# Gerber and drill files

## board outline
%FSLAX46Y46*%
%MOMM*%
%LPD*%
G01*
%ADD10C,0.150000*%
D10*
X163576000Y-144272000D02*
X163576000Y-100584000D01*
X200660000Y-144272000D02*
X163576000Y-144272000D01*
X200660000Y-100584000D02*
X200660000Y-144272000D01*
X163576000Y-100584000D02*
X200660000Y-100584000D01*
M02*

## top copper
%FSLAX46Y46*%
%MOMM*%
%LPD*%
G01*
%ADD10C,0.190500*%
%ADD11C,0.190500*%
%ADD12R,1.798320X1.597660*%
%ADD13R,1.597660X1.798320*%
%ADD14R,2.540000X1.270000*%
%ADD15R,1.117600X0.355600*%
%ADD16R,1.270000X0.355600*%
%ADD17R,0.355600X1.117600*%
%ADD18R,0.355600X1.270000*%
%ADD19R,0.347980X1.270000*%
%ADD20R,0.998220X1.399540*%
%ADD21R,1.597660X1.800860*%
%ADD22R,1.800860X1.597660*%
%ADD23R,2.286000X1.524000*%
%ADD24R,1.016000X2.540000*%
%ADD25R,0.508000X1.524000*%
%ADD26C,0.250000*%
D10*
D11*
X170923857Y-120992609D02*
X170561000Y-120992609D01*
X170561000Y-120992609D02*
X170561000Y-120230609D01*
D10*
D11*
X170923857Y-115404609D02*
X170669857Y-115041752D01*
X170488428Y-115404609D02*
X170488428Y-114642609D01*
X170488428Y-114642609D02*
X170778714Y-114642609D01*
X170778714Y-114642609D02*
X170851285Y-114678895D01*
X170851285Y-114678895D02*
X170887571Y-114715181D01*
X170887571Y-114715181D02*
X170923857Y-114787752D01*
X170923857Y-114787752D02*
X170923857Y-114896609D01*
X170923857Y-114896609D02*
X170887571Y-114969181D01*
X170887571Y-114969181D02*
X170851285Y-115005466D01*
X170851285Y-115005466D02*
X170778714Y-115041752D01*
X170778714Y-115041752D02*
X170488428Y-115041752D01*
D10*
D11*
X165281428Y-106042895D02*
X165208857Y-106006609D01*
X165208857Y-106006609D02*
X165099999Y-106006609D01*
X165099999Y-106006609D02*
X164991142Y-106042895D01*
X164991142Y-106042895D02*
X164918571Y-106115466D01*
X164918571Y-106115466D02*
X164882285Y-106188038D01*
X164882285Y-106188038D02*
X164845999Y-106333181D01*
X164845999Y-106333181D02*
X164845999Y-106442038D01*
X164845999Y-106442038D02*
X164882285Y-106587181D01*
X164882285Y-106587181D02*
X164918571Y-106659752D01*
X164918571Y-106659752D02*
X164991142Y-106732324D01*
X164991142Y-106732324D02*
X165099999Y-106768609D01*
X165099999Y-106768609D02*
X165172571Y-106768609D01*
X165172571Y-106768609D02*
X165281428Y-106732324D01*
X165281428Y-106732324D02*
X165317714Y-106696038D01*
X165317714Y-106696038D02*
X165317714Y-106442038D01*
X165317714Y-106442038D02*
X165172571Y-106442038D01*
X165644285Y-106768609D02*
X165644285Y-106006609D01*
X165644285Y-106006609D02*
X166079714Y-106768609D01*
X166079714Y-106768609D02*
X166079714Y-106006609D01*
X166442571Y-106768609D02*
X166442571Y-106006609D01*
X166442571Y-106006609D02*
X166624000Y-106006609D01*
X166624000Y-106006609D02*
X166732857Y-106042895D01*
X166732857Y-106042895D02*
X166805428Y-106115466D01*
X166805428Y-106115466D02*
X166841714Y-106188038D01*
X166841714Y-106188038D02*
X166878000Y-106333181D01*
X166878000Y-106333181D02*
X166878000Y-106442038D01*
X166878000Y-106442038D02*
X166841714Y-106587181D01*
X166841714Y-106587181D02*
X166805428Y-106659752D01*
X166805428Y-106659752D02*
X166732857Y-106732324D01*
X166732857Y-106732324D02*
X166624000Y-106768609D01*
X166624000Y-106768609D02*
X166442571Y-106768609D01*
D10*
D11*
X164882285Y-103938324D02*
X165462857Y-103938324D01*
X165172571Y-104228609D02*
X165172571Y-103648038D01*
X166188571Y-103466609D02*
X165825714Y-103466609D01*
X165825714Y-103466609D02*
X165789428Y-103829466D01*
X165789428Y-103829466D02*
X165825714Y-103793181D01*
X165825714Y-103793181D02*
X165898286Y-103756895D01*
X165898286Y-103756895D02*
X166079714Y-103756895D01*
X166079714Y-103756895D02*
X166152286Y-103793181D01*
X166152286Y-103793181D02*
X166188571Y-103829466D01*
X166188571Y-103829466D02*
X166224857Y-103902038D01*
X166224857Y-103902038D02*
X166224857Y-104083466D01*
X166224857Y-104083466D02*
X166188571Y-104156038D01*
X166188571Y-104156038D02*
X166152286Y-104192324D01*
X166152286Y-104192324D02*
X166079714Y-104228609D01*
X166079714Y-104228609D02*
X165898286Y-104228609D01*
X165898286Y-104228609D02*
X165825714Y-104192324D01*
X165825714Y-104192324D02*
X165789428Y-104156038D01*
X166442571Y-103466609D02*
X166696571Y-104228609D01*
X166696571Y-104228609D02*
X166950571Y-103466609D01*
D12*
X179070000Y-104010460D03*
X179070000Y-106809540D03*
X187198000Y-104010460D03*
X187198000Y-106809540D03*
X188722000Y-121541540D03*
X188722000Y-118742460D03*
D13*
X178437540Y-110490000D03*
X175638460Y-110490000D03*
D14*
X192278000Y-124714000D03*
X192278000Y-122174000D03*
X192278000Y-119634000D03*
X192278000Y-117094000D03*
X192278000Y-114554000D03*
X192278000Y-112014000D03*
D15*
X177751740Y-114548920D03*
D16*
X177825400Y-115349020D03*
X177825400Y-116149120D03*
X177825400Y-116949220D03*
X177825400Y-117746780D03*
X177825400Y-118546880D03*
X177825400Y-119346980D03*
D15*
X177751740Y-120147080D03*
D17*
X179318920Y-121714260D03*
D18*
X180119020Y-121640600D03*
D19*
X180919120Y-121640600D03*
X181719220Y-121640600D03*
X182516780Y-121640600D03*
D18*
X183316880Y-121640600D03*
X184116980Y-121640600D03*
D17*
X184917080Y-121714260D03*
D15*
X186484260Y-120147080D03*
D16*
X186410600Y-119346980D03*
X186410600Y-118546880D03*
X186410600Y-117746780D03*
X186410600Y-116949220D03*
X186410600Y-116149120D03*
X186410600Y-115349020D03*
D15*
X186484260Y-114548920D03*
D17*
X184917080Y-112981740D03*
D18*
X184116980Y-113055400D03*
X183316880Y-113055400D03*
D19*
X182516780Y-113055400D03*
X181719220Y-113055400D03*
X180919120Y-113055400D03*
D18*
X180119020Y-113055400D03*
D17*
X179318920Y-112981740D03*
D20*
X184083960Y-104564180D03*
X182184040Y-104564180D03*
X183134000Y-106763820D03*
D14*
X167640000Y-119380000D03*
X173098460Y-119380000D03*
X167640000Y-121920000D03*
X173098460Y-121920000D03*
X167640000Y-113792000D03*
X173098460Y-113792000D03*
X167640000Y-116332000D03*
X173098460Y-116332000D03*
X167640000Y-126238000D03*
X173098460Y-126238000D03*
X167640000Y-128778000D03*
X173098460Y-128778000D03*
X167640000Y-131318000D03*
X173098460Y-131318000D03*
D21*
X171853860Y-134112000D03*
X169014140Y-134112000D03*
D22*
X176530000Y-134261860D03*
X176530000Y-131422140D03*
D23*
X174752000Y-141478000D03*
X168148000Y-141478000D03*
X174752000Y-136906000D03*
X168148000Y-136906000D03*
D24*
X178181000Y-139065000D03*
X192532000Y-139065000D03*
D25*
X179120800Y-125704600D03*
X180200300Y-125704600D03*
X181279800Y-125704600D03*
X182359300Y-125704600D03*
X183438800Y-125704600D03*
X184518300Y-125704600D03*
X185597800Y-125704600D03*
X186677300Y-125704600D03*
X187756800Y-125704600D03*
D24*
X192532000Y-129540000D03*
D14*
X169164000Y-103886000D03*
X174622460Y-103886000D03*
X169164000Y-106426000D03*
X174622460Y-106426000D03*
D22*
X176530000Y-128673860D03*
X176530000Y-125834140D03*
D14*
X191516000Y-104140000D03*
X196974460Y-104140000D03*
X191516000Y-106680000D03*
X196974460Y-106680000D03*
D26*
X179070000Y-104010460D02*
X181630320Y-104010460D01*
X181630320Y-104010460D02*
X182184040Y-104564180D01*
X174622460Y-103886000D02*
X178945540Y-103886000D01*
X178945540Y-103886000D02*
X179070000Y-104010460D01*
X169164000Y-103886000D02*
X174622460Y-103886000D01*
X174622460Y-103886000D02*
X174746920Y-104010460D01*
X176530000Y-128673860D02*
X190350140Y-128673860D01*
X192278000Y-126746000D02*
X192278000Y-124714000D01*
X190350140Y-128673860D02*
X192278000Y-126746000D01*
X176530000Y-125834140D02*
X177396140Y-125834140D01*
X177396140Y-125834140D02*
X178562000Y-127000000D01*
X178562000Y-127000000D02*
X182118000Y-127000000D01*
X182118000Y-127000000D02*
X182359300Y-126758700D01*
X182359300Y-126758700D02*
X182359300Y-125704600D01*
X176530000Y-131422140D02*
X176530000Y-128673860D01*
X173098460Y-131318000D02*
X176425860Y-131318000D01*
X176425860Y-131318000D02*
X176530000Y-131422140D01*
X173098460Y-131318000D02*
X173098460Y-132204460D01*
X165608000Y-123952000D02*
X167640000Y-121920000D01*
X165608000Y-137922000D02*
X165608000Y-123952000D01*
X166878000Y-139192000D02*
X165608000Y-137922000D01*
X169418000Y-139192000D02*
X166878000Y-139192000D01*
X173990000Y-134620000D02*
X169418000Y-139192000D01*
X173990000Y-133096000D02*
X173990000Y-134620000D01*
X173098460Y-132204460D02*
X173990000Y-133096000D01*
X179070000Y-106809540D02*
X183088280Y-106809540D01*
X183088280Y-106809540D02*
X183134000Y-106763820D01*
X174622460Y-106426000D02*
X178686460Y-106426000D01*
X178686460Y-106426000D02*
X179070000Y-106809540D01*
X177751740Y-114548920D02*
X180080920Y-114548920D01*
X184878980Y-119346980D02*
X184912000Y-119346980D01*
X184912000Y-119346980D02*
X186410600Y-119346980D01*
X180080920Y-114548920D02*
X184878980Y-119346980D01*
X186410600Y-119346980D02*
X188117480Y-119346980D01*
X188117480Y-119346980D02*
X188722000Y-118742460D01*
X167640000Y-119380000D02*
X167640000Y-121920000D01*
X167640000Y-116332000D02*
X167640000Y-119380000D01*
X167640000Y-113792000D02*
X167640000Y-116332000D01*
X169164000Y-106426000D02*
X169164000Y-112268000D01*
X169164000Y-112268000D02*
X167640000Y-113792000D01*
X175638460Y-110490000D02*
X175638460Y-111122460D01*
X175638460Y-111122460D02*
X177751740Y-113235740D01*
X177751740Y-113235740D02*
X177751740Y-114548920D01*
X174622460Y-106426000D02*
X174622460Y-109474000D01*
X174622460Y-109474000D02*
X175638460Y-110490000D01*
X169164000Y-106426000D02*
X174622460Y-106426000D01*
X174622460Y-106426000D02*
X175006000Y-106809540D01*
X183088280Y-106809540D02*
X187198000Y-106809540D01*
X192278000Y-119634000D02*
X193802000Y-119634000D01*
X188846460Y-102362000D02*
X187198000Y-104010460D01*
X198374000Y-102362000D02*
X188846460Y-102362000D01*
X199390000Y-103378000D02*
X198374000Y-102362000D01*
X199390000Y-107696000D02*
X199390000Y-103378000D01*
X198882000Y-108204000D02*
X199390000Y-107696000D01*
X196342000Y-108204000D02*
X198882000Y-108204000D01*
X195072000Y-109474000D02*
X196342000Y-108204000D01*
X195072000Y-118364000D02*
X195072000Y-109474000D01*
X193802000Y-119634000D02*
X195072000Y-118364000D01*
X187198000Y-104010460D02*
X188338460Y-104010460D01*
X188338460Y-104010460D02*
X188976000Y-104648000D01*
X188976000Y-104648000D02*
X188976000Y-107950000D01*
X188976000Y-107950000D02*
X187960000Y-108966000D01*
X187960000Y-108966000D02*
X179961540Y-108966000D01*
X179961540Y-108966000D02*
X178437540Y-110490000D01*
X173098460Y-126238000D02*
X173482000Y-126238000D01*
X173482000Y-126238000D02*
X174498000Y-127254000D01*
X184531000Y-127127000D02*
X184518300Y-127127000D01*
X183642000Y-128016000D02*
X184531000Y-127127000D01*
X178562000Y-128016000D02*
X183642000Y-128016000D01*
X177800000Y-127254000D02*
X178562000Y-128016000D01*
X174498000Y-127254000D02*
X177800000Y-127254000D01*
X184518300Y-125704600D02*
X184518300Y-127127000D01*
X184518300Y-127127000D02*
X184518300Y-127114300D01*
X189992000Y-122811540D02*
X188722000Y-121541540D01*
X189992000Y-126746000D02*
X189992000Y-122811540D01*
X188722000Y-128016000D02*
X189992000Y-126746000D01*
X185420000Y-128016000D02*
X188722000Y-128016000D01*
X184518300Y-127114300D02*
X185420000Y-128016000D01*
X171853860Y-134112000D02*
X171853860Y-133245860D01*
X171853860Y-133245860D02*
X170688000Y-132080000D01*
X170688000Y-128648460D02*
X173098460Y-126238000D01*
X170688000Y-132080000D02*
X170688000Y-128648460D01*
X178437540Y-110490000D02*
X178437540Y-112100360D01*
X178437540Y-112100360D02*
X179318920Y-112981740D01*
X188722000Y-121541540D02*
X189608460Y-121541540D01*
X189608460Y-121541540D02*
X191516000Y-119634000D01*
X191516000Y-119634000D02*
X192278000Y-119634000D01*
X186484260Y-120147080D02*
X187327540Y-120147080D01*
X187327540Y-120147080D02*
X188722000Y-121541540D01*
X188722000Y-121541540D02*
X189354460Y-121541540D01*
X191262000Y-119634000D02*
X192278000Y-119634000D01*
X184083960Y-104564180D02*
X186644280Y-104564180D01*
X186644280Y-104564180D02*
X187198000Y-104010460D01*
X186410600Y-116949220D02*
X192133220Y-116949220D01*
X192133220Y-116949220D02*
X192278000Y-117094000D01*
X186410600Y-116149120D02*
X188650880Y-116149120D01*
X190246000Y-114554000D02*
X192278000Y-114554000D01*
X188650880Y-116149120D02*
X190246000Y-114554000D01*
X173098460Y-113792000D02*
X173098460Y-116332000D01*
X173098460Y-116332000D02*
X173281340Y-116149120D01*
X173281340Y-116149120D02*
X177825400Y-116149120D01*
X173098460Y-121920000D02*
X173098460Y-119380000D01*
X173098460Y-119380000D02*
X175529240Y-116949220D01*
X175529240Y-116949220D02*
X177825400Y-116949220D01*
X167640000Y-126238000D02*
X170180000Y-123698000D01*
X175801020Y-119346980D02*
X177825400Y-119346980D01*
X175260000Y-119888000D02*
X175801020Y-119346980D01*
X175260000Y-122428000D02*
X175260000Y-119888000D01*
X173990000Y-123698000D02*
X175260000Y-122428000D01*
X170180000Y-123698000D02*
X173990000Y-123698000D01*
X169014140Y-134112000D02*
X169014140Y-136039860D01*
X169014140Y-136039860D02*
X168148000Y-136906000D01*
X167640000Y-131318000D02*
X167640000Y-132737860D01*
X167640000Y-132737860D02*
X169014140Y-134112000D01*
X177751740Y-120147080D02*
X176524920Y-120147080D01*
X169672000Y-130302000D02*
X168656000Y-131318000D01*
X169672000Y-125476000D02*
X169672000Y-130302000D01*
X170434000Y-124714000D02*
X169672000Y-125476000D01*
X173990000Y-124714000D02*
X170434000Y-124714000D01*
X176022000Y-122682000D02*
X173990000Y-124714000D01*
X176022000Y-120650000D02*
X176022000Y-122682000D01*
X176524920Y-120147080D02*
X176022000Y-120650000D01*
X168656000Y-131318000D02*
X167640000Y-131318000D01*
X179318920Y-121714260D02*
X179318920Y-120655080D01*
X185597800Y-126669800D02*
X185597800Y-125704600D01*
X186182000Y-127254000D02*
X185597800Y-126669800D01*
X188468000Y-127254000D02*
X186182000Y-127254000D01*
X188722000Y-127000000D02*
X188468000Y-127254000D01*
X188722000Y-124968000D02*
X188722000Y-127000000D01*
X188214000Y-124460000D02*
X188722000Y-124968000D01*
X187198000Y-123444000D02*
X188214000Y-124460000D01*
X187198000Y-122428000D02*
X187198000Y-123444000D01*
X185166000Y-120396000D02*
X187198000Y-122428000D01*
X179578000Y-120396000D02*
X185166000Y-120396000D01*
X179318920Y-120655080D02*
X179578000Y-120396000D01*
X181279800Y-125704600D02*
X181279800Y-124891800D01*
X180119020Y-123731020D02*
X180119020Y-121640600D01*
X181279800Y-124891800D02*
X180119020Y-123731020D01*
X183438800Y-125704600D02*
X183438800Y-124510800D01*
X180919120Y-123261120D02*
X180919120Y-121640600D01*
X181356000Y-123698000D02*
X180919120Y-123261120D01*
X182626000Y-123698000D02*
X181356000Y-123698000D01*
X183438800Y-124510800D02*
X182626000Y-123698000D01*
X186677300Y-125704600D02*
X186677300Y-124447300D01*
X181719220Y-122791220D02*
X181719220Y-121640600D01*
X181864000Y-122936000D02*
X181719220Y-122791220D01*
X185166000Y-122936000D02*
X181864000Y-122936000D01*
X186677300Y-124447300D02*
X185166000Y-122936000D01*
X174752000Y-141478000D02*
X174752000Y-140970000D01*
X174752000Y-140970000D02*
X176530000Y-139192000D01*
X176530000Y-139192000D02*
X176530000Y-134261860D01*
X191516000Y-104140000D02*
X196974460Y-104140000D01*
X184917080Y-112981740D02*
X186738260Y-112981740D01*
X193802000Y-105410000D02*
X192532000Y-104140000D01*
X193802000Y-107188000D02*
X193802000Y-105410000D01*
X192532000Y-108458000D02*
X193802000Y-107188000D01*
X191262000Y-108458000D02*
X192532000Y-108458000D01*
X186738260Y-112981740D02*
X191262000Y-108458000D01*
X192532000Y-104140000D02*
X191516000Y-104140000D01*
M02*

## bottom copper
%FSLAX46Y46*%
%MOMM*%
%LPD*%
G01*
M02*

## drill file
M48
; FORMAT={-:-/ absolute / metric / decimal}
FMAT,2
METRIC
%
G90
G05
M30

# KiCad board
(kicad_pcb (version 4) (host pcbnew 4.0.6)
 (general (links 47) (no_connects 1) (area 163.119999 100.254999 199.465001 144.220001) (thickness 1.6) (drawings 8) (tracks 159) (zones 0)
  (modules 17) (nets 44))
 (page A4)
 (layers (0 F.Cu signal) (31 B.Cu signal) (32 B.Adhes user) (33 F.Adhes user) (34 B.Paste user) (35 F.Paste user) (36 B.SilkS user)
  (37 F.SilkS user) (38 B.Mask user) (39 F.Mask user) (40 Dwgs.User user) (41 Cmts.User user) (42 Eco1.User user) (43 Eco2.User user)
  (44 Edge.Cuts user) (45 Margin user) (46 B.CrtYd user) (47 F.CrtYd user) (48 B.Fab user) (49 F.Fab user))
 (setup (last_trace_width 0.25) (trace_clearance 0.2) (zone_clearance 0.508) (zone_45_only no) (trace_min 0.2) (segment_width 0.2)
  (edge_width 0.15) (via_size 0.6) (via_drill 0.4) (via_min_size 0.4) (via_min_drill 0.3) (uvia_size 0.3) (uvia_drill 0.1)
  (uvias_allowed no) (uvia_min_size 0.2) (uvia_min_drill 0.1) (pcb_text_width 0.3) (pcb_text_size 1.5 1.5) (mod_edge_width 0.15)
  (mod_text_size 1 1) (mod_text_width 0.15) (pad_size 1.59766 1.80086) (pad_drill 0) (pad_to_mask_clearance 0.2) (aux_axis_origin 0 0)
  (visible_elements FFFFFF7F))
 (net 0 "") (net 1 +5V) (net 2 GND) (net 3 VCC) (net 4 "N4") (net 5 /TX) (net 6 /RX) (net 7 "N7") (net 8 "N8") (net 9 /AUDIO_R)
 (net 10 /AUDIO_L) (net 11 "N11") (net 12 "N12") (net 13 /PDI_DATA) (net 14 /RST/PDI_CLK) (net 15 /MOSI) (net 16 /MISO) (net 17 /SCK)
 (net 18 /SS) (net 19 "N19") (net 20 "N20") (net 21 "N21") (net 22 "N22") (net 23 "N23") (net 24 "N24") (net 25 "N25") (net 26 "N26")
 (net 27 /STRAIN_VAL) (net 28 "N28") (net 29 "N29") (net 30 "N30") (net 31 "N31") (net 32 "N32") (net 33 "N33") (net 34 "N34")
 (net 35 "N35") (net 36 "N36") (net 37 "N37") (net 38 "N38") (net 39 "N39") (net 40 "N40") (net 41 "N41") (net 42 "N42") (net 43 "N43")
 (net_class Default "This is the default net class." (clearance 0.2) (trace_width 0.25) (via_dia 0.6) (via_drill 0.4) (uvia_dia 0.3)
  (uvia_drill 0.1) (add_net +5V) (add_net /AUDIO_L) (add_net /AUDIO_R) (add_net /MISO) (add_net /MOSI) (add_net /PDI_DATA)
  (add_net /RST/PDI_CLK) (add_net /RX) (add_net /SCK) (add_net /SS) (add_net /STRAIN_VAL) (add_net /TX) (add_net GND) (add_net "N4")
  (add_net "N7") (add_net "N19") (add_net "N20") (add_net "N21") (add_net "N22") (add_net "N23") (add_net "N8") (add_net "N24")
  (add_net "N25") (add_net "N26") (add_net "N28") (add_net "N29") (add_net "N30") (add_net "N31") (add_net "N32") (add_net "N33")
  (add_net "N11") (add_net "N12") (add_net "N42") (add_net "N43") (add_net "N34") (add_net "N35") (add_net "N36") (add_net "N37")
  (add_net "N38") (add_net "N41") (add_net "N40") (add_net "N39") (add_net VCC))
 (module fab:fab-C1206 (layer F.Cu) (at 179.07 105.41 270)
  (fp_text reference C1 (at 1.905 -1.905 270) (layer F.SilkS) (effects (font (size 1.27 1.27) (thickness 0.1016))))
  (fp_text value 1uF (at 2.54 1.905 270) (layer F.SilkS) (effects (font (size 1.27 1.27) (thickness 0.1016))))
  (pad 1 smd rect (at -1.39954 0 270) (size 1.59766 1.79832) (layers F.Cu F.Paste F.Mask) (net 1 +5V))
  (pad 2 smd rect (at 1.39954 0 270) (size 1.59766 1.79832) (layers F.Cu F.Paste F.Mask) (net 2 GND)))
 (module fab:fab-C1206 (layer F.Cu) (at 187.198 105.41 270)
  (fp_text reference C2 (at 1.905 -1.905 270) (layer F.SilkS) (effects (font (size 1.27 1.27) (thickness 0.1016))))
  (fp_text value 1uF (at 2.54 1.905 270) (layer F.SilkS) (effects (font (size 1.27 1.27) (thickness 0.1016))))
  (pad 1 smd rect (at -1.39954 0 270) (size 1.59766 1.79832) (layers F.Cu F.Paste F.Mask) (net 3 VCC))
  (pad 2 smd rect (at 1.39954 0 270) (size 1.59766 1.79832) (layers F.Cu F.Paste F.Mask) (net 2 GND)))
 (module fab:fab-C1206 (layer F.Cu) (at 188.722 120.142 90)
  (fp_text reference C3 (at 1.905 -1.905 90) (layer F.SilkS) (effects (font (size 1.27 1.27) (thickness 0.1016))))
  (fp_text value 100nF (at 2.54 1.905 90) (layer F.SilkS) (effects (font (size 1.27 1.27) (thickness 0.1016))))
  (pad 1 smd rect (at -1.39954 0 90) (size 1.59766 1.79832) (layers F.Cu F.Paste F.Mask) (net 3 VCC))
  (pad 2 smd rect (at 1.39954 0 90) (size 1.59766 1.79832) (layers F.Cu F.Paste F.Mask) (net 2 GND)))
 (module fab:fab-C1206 (layer F.Cu) (at 177.038 110.49 180)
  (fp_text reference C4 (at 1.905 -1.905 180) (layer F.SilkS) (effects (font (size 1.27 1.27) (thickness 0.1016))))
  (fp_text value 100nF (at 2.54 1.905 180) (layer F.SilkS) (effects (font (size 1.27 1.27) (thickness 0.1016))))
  (pad 1 smd rect (at -1.39954 0 180) (size 1.59766 1.79832) (layers F.Cu F.Paste F.Mask) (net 3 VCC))
  (pad 2 smd rect (at 1.39954 0 180) (size 1.59766 1.79832) (layers F.Cu F.Paste F.Mask) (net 2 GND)))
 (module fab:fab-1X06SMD (layer F.Cu) (at 192.278 118.364 180)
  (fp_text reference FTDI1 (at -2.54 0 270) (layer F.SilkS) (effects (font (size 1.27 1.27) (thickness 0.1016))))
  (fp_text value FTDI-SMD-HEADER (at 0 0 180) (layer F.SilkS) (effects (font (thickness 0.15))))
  (pad 1 smd rect (at 0 -6.35 180) (size 2.54 1.27) (layers F.Cu F.Paste F.Mask) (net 2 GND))
  (pad 2 smd rect (at 0 -3.81 180) (size 2.54 1.27) (layers F.Cu F.Paste F.Mask) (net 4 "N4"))
  (pad 3 smd rect (at 0 -1.27 180) (size 2.54 1.27) (layers F.Cu F.Paste F.Mask) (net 3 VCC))
  (pad 4 smd rect (at 0 1.27 180) (size 2.54 1.27) (layers F.Cu F.Paste F.Mask) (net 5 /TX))
  (pad 5 smd rect (at 0 3.81 180) (size 2.54 1.27) (layers F.Cu F.Paste F.Mask) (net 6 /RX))
  (pad 6 smd rect (at 0 6.35 180) (size 2.54 1.27) (layers F.Cu F.Paste F.Mask) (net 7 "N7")))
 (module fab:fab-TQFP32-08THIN (layer F.Cu) (at 182.118 117.348)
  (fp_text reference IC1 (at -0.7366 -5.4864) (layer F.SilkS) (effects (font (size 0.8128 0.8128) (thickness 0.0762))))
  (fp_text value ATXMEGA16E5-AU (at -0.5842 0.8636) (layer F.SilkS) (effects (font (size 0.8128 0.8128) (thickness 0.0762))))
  (pad 1 smd rect (at -4.36626 -2.79908) (size 1.1176 0.3556) (layers F.Cu F.Paste F.Mask) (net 2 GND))
  (pad 2 smd rect (at -4.2926 -1.99898) (size 1.27 0.3556) (layers F.Cu F.Paste F.Mask) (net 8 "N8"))
  (pad 3 smd rect (at -4.2926 -1.19888) (size 1.27 0.3556) (layers F.Cu F.Paste F.Mask) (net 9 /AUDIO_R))
  (pad 4 smd rect (at -4.2926 -0.39878) (size 1.27 0.3556) (layers F.Cu F.Paste F.Mask) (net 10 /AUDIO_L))
  (pad 5 smd rect (at -4.2926 0.39878) (size 1.27 0.3556) (layers F.Cu F.Paste F.Mask) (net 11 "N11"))
  (pad 6 smd rect (at -4.2926 1.19888) (size 1.27 0.3556) (layers F.Cu F.Paste F.Mask) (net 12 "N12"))
  (pad 7 smd rect (at -4.2926 1.99898) (size 1.27 0.3556) (layers F.Cu F.Paste F.Mask) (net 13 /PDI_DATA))
  (pad 8 smd rect (at -4.36626 2.79908) (size 1.1176 0.3556) (layers F.Cu F.Paste F.Mask) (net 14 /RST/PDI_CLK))
  (pad 9 smd rect (at -2.79908 4.36626) (size 0.3556 1.1176) (layers F.Cu F.Paste F.Mask) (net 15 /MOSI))
  (pad 10 smd rect (at -1.99898 4.2926) (size 0.3556 1.27) (layers F.Cu F.Paste F.Mask) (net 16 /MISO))
  (pad 11 smd rect (at -1.19888 4.2926) (size 0.34798 1.27) (layers F.Cu F.Paste F.Mask) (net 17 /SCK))
  (pad 12 smd rect (at -0.39878 4.2926) (size 0.34798 1.27) (layers F.Cu F.Paste F.Mask) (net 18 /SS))
  (pad 13 smd rect (at 0.39878 4.2926) (size 0.34798 1.27) (layers F.Cu F.Paste F.Mask) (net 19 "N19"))
  (pad 14 smd rect (at 1.19888 4.2926) (size 0.3556 1.27) (layers F.Cu F.Paste F.Mask) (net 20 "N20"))
  (pad 15 smd rect (at 1.99898 4.2926) (size 0.3556 1.27) (layers F.Cu F.Paste F.Mask) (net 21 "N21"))
  (pad 16 smd rect (at 2.79908 4.36626) (size 0.3556 1.1176) (layers F.Cu F.Paste F.Mask) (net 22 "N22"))
  (pad 17 smd rect (at 4.36626 2.79908) (size 1.1176 0.3556) (layers F.Cu F.Paste F.Mask) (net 3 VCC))
  (pad 18 smd rect (at 4.2926 1.99898) (size 1.27 0.3556) (layers F.Cu F.Paste F.Mask) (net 2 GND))
  (pad 19 smd rect (at 4.2926 1.19888) (size 1.27 0.3556) (layers F.Cu F.Paste F.Mask) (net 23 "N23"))
  (pad 20 smd rect (at 4.2926 0.39878) (size 1.27 0.3556) (layers F.Cu F.Paste F.Mask) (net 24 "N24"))
  (pad 21 smd rect (at 4.2926 -0.39878) (size 1.27 0.3556) (layers F.Cu F.Paste F.Mask) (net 5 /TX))
  (pad 22 smd rect (at 4.2926 -1.19888) (size 1.27 0.3556) (layers F.Cu F.Paste F.Mask) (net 6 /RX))
  (pad 23 smd rect (at 4.2926 -1.99898) (size 1.27 0.3556) (layers F.Cu F.Paste F.Mask) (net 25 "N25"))
  (pad 24 smd rect (at 4.36626 -2.79908) (size 1.1176 0.3556) (layers F.Cu F.Paste F.Mask) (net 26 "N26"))
  (pad 25 smd rect (at 2.79908 -4.36626) (size 0.3556 1.1176) (layers F.Cu F.Paste F.Mask) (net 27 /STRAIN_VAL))
  (pad 26 smd rect (at 1.99898 -4.2926) (size 0.3556 1.27) (layers F.Cu F.Paste F.Mask) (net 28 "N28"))
  (pad 27 smd rect (at 1.19888 -4.2926) (size 0.3556 1.27) (layers F.Cu F.Paste F.Mask) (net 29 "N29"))
  (pad 28 smd rect (at 0.39878 -4.2926) (size 0.34798 1.27) (layers F.Cu F.Paste F.Mask) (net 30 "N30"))
  (pad 29 smd rect (at -0.39878 -4.2926) (size 0.34798 1.27) (layers F.Cu F.Paste F.Mask) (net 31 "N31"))
  (pad 30 smd rect (at -1.19888 -4.2926) (size 0.34798 1.27) (layers F.Cu F.Paste F.Mask) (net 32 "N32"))
  (pad 31 smd rect (at -1.99898 -4.2926) (size 0.3556 1.27) (layers F.Cu F.Paste F.Mask) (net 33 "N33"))
  (pad 32 smd rect (at -2.79908 -4.36626) (size 0.3556 1.1176) (layers F.Cu F.Paste F.Mask) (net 3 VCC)))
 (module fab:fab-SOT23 (layer F.Cu) (at 183.134 105.664 180)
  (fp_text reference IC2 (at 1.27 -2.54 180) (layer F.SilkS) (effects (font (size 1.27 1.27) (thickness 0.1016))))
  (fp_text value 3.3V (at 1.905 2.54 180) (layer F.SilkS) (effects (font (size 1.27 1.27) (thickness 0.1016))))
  (pad 1 smd rect (at -0.94996 1.09982 180) (size 0.99822 1.39954) (layers F.Cu F.Paste F.Mask) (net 3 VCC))
  (pad 2 smd rect (at 0.94996 1.09982 180) (size 0.99822 1.39954) (layers F.Cu F.Paste F.Mask) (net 1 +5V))
  (pad 3 smd rect (at 0 -1.09982 180) (size 0.99822 1.39954) (layers F.Cu F.Paste F.Mask) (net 2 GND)))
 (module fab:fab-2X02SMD (layer F.Cu) (at 170.18 120.65)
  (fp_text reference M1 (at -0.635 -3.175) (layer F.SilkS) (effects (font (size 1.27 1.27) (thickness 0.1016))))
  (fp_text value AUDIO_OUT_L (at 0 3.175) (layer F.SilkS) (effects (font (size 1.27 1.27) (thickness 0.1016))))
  (pad 1 smd rect (at -2.54 -1.27) (size 2.54 1.27) (layers F.Cu F.Paste F.Mask) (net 2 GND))
  (pad 2 smd rect (at 2.91846 -1.27) (size 2.54 1.27) (layers F.Cu F.Paste F.Mask) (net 10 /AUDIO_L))
  (pad 3 smd rect (at -2.54 1.27) (size 2.54 1.27) (layers F.Cu F.Paste F.Mask) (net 2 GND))
  (pad 4 smd rect (at 2.91846 1.27) (size 2.54 1.27) (layers F.Cu F.Paste F.Mask) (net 10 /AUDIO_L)))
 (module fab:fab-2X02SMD (layer F.Cu) (at 170.18 115.062)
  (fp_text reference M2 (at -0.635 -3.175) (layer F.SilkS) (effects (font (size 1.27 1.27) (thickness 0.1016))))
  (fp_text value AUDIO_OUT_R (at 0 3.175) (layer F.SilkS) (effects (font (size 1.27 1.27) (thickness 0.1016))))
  (pad 1 smd rect (at -2.54 -1.27) (size 2.54 1.27) (layers F.Cu F.Paste F.Mask) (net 2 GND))
  (pad 2 smd rect (at 2.91846 -1.27) (size 2.54 1.27) (layers F.Cu F.Paste F.Mask) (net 9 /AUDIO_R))
  (pad 3 smd rect (at -2.54 1.27) (size 2.54 1.27) (layers F.Cu F.Paste F.Mask) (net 2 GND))
  (pad 4 smd rect (at 2.91846 1.27) (size 2.54 1.27) (layers F.Cu F.Paste F.Mask) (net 9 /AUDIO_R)))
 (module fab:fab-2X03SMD (layer F.Cu) (at 170.18 128.778)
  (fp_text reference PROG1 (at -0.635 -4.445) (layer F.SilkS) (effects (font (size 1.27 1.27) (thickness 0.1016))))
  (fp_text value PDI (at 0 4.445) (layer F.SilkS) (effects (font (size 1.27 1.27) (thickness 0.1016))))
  (pad 1 smd rect (at -2.54 -2.54) (size 2.54 1.27) (layers F.Cu F.Paste F.Mask) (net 13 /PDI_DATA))
  (pad 2 smd rect (at 2.91846 -2.54) (size 2.54 1.27) (layers F.Cu F.Paste F.Mask) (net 3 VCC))
  (pad 3 smd rect (at -2.54 0) (size 2.54 1.27) (layers F.Cu F.Paste F.Mask) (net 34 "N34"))
  (pad 4 smd rect (at 2.91846 0) (size 2.54 1.27) (layers F.Cu F.Paste F.Mask) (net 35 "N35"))
  (pad 5 smd rect (at -2.54 2.54) (size 2.54 1.27) (layers F.Cu F.Paste F.Mask) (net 14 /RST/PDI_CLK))
  (pad 6 smd rect (at 2.91846 2.54) (size 2.54 1.27) (layers F.Cu F.Paste F.Mask) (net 2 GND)))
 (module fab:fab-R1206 (layer F.Cu) (at 170.434 134.112 180)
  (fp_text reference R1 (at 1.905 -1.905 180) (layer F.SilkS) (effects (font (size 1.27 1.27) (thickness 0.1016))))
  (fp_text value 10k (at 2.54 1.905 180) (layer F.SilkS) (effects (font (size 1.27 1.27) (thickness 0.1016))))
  (pad 1 smd rect (at -1.41986 0 180) (size 1.59766 1.80086) (layers F.Cu F.Paste F.Mask) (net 3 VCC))
  (pad 2 smd rect (at 1.41986 0 180) (size 1.59766 1.80086) (layers F.Cu F.Paste F.Mask) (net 14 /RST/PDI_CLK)))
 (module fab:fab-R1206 (layer F.Cu) (at 176.53 132.842 90)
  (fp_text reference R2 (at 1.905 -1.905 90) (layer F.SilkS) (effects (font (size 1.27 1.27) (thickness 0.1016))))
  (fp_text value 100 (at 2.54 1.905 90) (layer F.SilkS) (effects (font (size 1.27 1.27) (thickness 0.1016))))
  (pad 1 smd rect (at -1.41986 0 90) (size 1.59766 1.80086) (layers F.Cu F.Paste F.Mask) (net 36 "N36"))
  (pad 2 smd rect (at 1.41986 0 90) (size 1.59766 1.80086) (layers F.Cu F.Paste F.Mask) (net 2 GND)))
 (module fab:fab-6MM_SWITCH (layer F.Cu) (at 171.45 139.192 180)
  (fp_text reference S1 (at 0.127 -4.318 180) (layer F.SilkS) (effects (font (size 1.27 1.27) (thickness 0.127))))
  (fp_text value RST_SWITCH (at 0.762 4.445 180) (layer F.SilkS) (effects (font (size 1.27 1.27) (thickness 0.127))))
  (pad 1 smd rect (at -3.302 -2.286 180) (size 2.286 1.524) (layers F.Cu F.Paste F.Mask) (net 36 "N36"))
  (pad 2 smd rect (at 3.302 -2.286 180) (size 2.286 1.524) (layers F.Cu F.Paste F.Mask) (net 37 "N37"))
  (pad 3 smd rect (at -3.302 2.286 180) (size 2.286 1.524) (layers F.Cu F.Paste F.Mask) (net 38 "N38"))
  (pad 4 smd rect (at 3.302 2.286 180) (size 2.286 1.524) (layers F.Cu F.Paste F.Mask) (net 14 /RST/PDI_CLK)))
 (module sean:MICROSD (layer F.Cu) (at 184.912 134.112)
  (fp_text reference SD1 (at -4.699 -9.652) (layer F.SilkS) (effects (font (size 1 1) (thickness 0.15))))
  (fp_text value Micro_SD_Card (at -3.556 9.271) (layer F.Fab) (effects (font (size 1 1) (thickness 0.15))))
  (pad SHEI smd rect (at -6.731 4.953) (size 1.016 2.54) (layers F.Cu F.Paste F.Mask))
  (pad SHEI smd rect (at 7.62 4.953) (size 1.016 2.54) (layers F.Cu F.Paste F.Mask))
  (pad 9 smd rect (at -5.7912 -8.4074) (size 0.508 1.524) (layers F.Cu F.Paste F.Mask) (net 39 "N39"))
  (pad 8 smd rect (at -4.7117 -8.4074) (size 0.508 1.524) (layers F.Cu F.Paste F.Mask) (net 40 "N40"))
  (pad 7 smd rect (at -3.6322 -8.4074) (size 0.508 1.524) (layers F.Cu F.Paste F.Mask) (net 16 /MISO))
  (pad 6 smd rect (at -2.5527 -8.4074) (size 0.508 1.524) (layers F.Cu F.Paste F.Mask) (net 2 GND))
  (pad 5 smd rect (at -1.4732 -8.4074) (size 0.508 1.524) (layers F.Cu F.Paste F.Mask) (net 17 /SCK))
  (pad 4 smd rect (at -0.3937 -8.4074) (size 0.508 1.524) (layers F.Cu F.Paste F.Mask) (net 3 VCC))
  (pad 3 smd rect (at 0.6858 -8.4074) (size 0.508 1.524) (layers F.Cu F.Paste F.Mask) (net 15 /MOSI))
  (pad 2 smd rect (at 1.7653 -8.4074) (size 0.508 1.524) (layers F.Cu F.Paste F.Mask) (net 18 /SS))
  (pad 1 smd rect (at 2.8448 -8.4074) (size 0.508 1.524) (layers F.Cu F.Paste F.Mask) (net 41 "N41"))
  (pad SHEI smd rect (at 7.62 -4.572) (size 1.016 2.54) (layers F.Cu F.Paste F.Mask)))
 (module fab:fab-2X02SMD (layer F.Cu) (at 171.704 105.156)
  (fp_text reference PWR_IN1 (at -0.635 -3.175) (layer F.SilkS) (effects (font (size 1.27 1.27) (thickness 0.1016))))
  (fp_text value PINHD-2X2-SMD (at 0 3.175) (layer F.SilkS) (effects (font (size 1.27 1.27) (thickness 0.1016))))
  (pad 1 smd rect (at -2.54 -1.27) (size 2.54 1.27) (layers F.Cu F.Paste F.Mask) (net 1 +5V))
  (pad 2 smd rect (at 2.91846 -1.27) (size 2.54 1.27) (layers F.Cu F.Paste F.Mask) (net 1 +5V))
  (pad 3 smd rect (at -2.54 1.27) (size 2.54 1.27) (layers F.Cu F.Paste F.Mask) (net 2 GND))
  (pad 4 smd rect (at 2.91846 1.27) (size 2.54 1.27) (layers F.Cu F.Paste F.Mask) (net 2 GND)))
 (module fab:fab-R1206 (layer F.Cu) (at 176.53 127.254 90)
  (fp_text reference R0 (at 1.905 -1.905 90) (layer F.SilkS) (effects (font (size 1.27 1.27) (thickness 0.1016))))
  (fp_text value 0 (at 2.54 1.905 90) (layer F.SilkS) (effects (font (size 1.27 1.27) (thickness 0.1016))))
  (pad 1 smd rect (at -1.41986 0 90) (size 1.59766 1.80086) (layers F.Cu F.Paste F.Mask) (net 2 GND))
  (pad 2 smd rect (at 1.41986 0 90) (size 1.59766 1.80086) (layers F.Cu F.Paste F.Mask) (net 2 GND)))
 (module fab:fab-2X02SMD (layer F.Cu) (at 194.056 105.41)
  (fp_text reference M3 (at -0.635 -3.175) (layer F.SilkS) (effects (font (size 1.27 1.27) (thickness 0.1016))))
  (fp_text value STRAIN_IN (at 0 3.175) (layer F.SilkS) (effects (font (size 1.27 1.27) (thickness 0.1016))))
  (pad 1 smd rect (at -2.54 -1.27) (size 2.54 1.27) (layers F.Cu F.Paste F.Mask) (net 27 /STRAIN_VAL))
  (pad 2 smd rect (at 2.91846 -1.27) (size 2.54 1.27) (layers F.Cu F.Paste F.Mask) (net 27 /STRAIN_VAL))
  (pad 3 smd rect (at -2.54 1.27) (size 2.54 1.27) (layers F.Cu F.Paste F.Mask) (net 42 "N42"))
  (pad 4 smd rect (at 2.91846 1.27) (size 2.54 1.27) (layers F.Cu F.Paste F.Mask) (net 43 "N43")))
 (gr_line (start 163.576 144.272) (end 163.576 100.584) (angle 90) (layer Edge.Cuts) (width 0.15))
 (gr_line (start 200.66 144.272) (end 163.576 144.272) (angle 90) (layer Edge.Cuts) (width 0.15))
 (gr_line (start 200.66 100.584) (end 200.66 144.272) (angle 90) (layer Edge.Cuts) (width 0.15))
 (gr_line (start 163.576 100.584) (end 200.66 100.584) (angle 90) (layer Edge.Cuts) (width 0.15))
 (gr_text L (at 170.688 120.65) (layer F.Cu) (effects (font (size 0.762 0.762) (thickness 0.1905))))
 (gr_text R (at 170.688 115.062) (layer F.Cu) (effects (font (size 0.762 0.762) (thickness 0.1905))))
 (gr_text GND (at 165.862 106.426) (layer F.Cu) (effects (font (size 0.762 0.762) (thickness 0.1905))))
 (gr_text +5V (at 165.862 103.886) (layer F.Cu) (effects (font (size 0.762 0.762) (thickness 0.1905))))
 (segment (start 179.07 104.01046) (end 181.63032 104.01046) (width 0.25) (layer F.Cu) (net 1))
 (segment (start 181.63032 104.01046) (end 182.18404 104.56418) (width 0.25) (layer F.Cu) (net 1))
 (segment (start 174.62246 103.886) (end 178.94554 103.886) (width 0.25) (layer F.Cu) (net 1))
 (segment (start 178.94554 103.886) (end 179.07 104.01046) (width 0.25) (layer F.Cu) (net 1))
 (segment (start 169.164 103.886) (end 174.62246 103.886) (width 0.25) (layer F.Cu) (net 1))
 (segment (start 174.62246 103.886) (end 174.74692 104.01046) (width 0.25) (layer F.Cu) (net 1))
 (segment (start 176.53 128.67386) (end 190.35014 128.67386) (width 0.25) (layer F.Cu) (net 2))
 (segment (start 192.278 126.746) (end 192.278 124.714) (width 0.25) (layer F.Cu) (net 2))
 (segment (start 190.35014 128.67386) (end 192.278 126.746) (width 0.25) (layer F.Cu) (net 2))
 (segment (start 176.53 125.83414) (end 177.39614 125.83414) (width 0.25) (layer F.Cu) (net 2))
 (segment (start 177.39614 125.83414) (end 178.562 127) (width 0.25) (layer F.Cu) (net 2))
 (segment (start 178.562 127) (end 182.118 127) (width 0.25) (layer F.Cu) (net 2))
 (segment (start 182.118 127) (end 182.3593 126.7587) (width 0.25) (layer F.Cu) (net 2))
 (segment (start 182.3593 126.7587) (end 182.3593 125.7046) (width 0.25) (layer F.Cu) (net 2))
 (segment (start 176.53 131.42214) (end 176.53 128.67386) (width 0.25) (layer F.Cu) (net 2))
 (segment (start 173.09846 131.318) (end 176.42586 131.318) (width 0.25) (layer F.Cu) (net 2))
 (segment (start 176.42586 131.318) (end 176.53 131.42214) (width 0.25) (layer F.Cu) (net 2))
 (segment (start 173.09846 131.318) (end 173.09846 132.20446) (width 0.25) (layer F.Cu) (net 2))
 (segment (start 165.608 123.952) (end 167.64 121.92) (width 0.25) (layer F.Cu) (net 2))
 (segment (start 165.608 137.922) (end 165.608 123.952) (width 0.25) (layer F.Cu) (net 2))
 (segment (start 166.878 139.192) (end 165.608 137.922) (width 0.25) (layer F.Cu) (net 2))
 (segment (start 169.418 139.192) (end 166.878 139.192) (width 0.25) (layer F.Cu) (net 2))
 (segment (start 173.99 134.62) (end 169.418 139.192) (width 0.25) (layer F.Cu) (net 2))
 (segment (start 173.99 133.096) (end 173.99 134.62) (width 0.25) (layer F.Cu) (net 2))
 (segment (start 173.09846 132.20446) (end 173.99 133.096) (width 0.25) (layer F.Cu) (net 2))
 (segment (start 179.07 106.80954) (end 183.08828 106.80954) (width 0.25) (layer F.Cu) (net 2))
 (segment (start 183.08828 106.80954) (end 183.134 106.76382) (width 0.25) (layer F.Cu) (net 2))
 (segment (start 174.62246 106.426) (end 178.68646 106.426) (width 0.25) (layer F.Cu) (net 2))
 (segment (start 178.68646 106.426) (end 179.07 106.80954) (width 0.25) (layer F.Cu) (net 2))
 (segment (start 177.75174 114.54892) (end 180.08092 114.54892) (width 0.25) (layer F.Cu) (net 2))
 (segment (start 184.87898 119.34698) (end 184.912 119.34698) (width 0.25) (layer F.Cu) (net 2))
 (segment (start 184.912 119.34698) (end 186.4106 119.34698) (width 0.25) (layer F.Cu) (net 2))
 (segment (start 180.08092 114.54892) (end 184.87898 119.34698) (width 0.25) (layer F.Cu) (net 2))
 (segment (start 186.4106 119.34698) (end 188.11748 119.34698) (width 0.25) (layer F.Cu) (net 2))
 (segment (start 188.11748 119.34698) (end 188.722 118.74246) (width 0.25) (layer F.Cu) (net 2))
 (segment (start 167.64 119.38) (end 167.64 121.92) (width 0.25) (layer F.Cu) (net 2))
 (segment (start 167.64 116.332) (end 167.64 119.38) (width 0.25) (layer F.Cu) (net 2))
 (segment (start 167.64 113.792) (end 167.64 116.332) (width 0.25) (layer F.Cu) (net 2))
 (segment (start 169.164 106.426) (end 169.164 112.268) (width 0.25) (layer F.Cu) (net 2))
 (segment (start 169.164 112.268) (end 167.64 113.792) (width 0.25) (layer F.Cu) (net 2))
 (segment (start 175.63846 110.49) (end 175.63846 111.12246) (width 0.25) (layer F.Cu) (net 2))
 (segment (start 175.63846 111.12246) (end 177.75174 113.23574) (width 0.25) (layer F.Cu) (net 2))
 (segment (start 177.75174 113.23574) (end 177.75174 114.54892) (width 0.25) (layer F.Cu) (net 2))
 (segment (start 174.62246 106.426) (end 174.62246 109.474) (width 0.25) (layer F.Cu) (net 2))
 (segment (start 174.62246 109.474) (end 175.63846 110.49) (width 0.25) (layer F.Cu) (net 2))
 (segment (start 169.164 106.426) (end 174.62246 106.426) (width 0.25) (layer F.Cu) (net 2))
 (segment (start 174.62246 106.426) (end 175.006 106.80954) (width 0.25) (layer F.Cu) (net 2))
 (segment (start 183.08828 106.80954) (end 187.198 106.80954) (width 0.25) (layer F.Cu) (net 2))
 (segment (start 192.278 119.634) (end 193.802 119.634) (width 0.25) (layer F.Cu) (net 3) (status 400000))
 (segment (start 188.84646 102.362) (end 187.198 104.01046) (width 0.25) (layer F.Cu) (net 3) (status 800000))
 (segment (start 198.374 102.362) (end 188.84646 102.362) (width 0.25) (layer F.Cu) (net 3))
 (segment (start 199.39 103.378) (end 198.374 102.362) (width 0.25) (layer F.Cu) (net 3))
 (segment (start 199.39 107.696) (end 199.39 103.378) (width 0.25) (layer F.Cu) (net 3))
 (segment (start 198.882 108.204) (end 199.39 107.696) (width 0.25) (layer F.Cu) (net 3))
 (segment (start 196.342 108.204) (end 198.882 108.204) (width 0.25) (layer F.Cu) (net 3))
 (segment (start 195.072 109.474) (end 196.342 108.204) (width 0.25) (layer F.Cu) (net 3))
 (segment (start 195.072 118.364) (end 195.072 109.474) (width 0.25) (layer F.Cu) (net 3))
 (segment (start 193.802 119.634) (end 195.072 118.364) (width 0.25) (layer F.Cu) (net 3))
 (segment (start 187.198 104.01046) (end 188.33846 104.01046) (width 0.25) (layer F.Cu) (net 3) (status 400000))
 (segment (start 188.33846 104.01046) (end 188.976 104.648) (width 0.25) (layer F.Cu) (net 3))
 (segment (start 188.976 104.648) (end 188.976 107.95) (width 0.25) (layer F.Cu) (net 3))
 (segment (start 188.976 107.95) (end 187.96 108.966) (width 0.25) (layer F.Cu) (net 3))
 (segment (start 187.96 108.966) (end 179.96154 108.966) (width 0.25) (layer F.Cu) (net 3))
 (segment (start 179.96154 108.966) (end 178.43754 110.49) (width 0.25) (layer F.Cu) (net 3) (status 800000))
 (segment (start 173.09846 126.238) (end 173.482 126.238) (width 0.25) (layer F.Cu) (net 3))
 (segment (start 173.482 126.238) (end 174.498 127.254) (width 0.25) (layer F.Cu) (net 3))
 (segment (start 184.531 127.127) (end 184.5183 127.127) (width 0.25) (layer F.Cu) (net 3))
 (segment (start 183.642 128.016) (end 184.531 127.127) (width 0.25) (layer F.Cu) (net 3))
 (segment (start 178.562 128.016) (end 183.642 128.016) (width 0.25) (layer F.Cu) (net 3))
 (segment (start 177.8 127.254) (end 178.562 128.016) (width 0.25) (layer F.Cu) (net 3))
 (segment (start 174.498 127.254) (end 177.8 127.254) (width 0.25) (layer F.Cu) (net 3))
 (segment (start 184.5183 125.7046) (end 184.5183 127.127) (width 0.25) (layer F.Cu) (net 3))
 (segment (start 184.5183 127.127) (end 184.5183 127.1143) (width 0.25) (layer F.Cu) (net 3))
 (segment (start 189.992 122.81154) (end 188.722 121.54154) (width 0.25) (layer F.Cu) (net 3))
 (segment (start 189.992 126.746) (end 189.992 122.81154) (width 0.25) (layer F.Cu) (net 3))
 (segment (start 188.722 128.016) (end 189.992 126.746) (width 0.25) (layer F.Cu) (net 3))
 (segment (start 185.42 128.016) (end 188.722 128.016) (width 0.25) (layer F.Cu) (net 3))
 (segment (start 184.5183 127.1143) (end 185.42 128.016) (width 0.25) (layer F.Cu) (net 3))
 (segment (start 171.85386 134.112) (end 171.85386 133.24586) (width 0.25) (layer F.Cu) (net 3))
 (segment (start 171.85386 133.24586) (end 170.688 132.08) (width 0.25) (layer F.Cu) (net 3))
 (segment (start 170.688 128.64846) (end 173.09846 126.238) (width 0.25) (layer F.Cu) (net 3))
 (segment (start 170.688 132.08) (end 170.688 128.64846) (width 0.25) (layer F.Cu) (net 3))
 (segment (start 178.43754 110.49) (end 178.43754 112.10036) (width 0.25) (layer F.Cu) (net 3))
 (segment (start 178.43754 112.10036) (end 179.31892 112.98174) (width 0.25) (layer F.Cu) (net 3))
 (segment (start 188.722 121.54154) (end 189.60846 121.54154) (width 0.25) (layer F.Cu) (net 3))
 (segment (start 189.60846 121.54154) (end 191.516 119.634) (width 0.25) (layer F.Cu) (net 3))
 (segment (start 191.516 119.634) (end 192.278 119.634) (width 0.25) (layer F.Cu) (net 3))
 (segment (start 186.48426 120.14708) (end 187.32754 120.14708) (width 0.25) (layer F.Cu) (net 3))
 (segment (start 187.32754 120.14708) (end 188.722 121.54154) (width 0.25) (layer F.Cu) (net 3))
 (segment (start 188.722 121.54154) (end 189.35446 121.54154) (width 0.25) (layer F.Cu) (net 3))
 (segment (start 191.262 119.634) (end 192.278 119.634) (width 0.25) (layer F.Cu) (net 3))
 (segment (start 184.08396 104.56418) (end 186.64428 104.56418) (width 0.25) (layer F.Cu) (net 3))
 (segment (start 186.64428 104.56418) (end 187.198 104.01046) (width 0.25) (layer F.Cu) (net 3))
 (segment (start 186.4106 116.94922) (end 192.13322 116.94922) (width 0.25) (layer F.Cu) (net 5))
 (segment (start 192.13322 116.94922) (end 192.278 117.094) (width 0.25) (layer F.Cu) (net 5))
 (segment (start 186.4106 116.14912) (end 188.65088 116.14912) (width 0.25) (layer F.Cu) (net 6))
 (segment (start 190.246 114.554) (end 192.278 114.554) (width 0.25) (layer F.Cu) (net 6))
 (segment (start 188.65088 116.14912) (end 190.246 114.554) (width 0.25) (layer F.Cu) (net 6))
 (segment (start 173.09846 113.792) (end 173.09846 116.332) (width 0.25) (layer F.Cu) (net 9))
 (segment (start 173.09846 116.332) (end 173.28134 116.14912) (width 0.25) (layer F.Cu) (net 9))
 (segment (start 173.28134 116.14912) (end 177.8254 116.14912) (width 0.25) (layer F.Cu) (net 9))
 (segment (start 173.09846 121.92) (end 173.09846 119.38) (width 0.25) (layer F.Cu) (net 10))
 (segment (start 173.09846 119.38) (end 175.52924 116.94922) (width 0.25) (layer F.Cu) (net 10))
 (segment (start 175.52924 116.94922) (end 177.8254 116.94922) (width 0.25) (layer F.Cu) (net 10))
 (segment (start 167.64 126.238) (end 170.18 123.698) (width 0.25) (layer F.Cu) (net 13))
 (segment (start 175.80102 119.34698) (end 177.8254 119.34698) (width 0.25) (layer F.Cu) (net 13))
 (segment (start 175.26 119.888) (end 175.80102 119.34698) (width 0.25) (layer F.Cu) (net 13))
 (segment (start 175.26 122.428) (end 175.26 119.888) (width 0.25) (layer F.Cu) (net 13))
 (segment (start 173.99 123.698) (end 175.26 122.428) (width 0.25) (layer F.Cu) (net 13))
 (segment (start 170.18 123.698) (end 173.99 123.698) (width 0.25) (layer F.Cu) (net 13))
 (segment (start 169.01414 134.112) (end 169.01414 136.03986) (width 0.25) (layer F.Cu) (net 14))
 (segment (start 169.01414 136.03986) (end 168.148 136.906) (width 0.25) (layer F.Cu) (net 14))
 (segment (start 167.64 131.318) (end 167.64 132.73786) (width 0.25) (layer F.Cu) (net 14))
 (segment (start 167.64 132.73786) (end 169.01414 134.112) (width 0.25) (layer F.Cu) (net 14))
 (segment (start 177.75174 120.14708) (end 176.52492 120.14708) (width 0.25) (layer F.Cu) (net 14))
 (segment (start 169.672 130.302) (end 168.656 131.318) (width 0.25) (layer F.Cu) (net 14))
 (segment (start 169.672 125.476) (end 169.672 130.302) (width 0.25) (layer F.Cu) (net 14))
 (segment (start 170.434 124.714) (end 169.672 125.476) (width 0.25) (layer F.Cu) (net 14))
 (segment (start 173.99 124.714) (end 170.434 124.714) (width 0.25) (layer F.Cu) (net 14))
 (segment (start 176.022 122.682) (end 173.99 124.714) (width 0.25) (layer F.Cu) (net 14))
 (segment (start 176.022 120.65) (end 176.022 122.682) (width 0.25) (layer F.Cu) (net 14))
 (segment (start 176.52492 120.14708) (end 176.022 120.65) (width 0.25) (layer F.Cu) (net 14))
 (segment (start 168.656 131.318) (end 167.64 131.318) (width 0.25) (layer F.Cu) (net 14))
 (segment (start 179.31892 121.71426) (end 179.31892 120.65508) (width 0.25) (layer F.Cu) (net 15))
 (segment (start 185.5978 126.6698) (end 185.5978 125.7046) (width 0.25) (layer F.Cu) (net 15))
 (segment (start 186.182 127.254) (end 185.5978 126.6698) (width 0.25) (layer F.Cu) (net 15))
 (segment (start 188.468 127.254) (end 186.182 127.254) (width 0.25) (layer F.Cu) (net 15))
 (segment (start 188.722 127) (end 188.468 127.254) (width 0.25) (layer F.Cu) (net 15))
 (segment (start 188.722 124.968) (end 188.722 127) (width 0.25) (layer F.Cu) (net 15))
 (segment (start 188.214 124.46) (end 188.722 124.968) (width 0.25) (layer F.Cu) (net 15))
 (segment (start 187.198 123.444) (end 188.214 124.46) (width 0.25) (layer F.Cu) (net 15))
 (segment (start 187.198 122.428) (end 187.198 123.444) (width 0.25) (layer F.Cu) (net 15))
 (segment (start 185.166 120.396) (end 187.198 122.428) (width 0.25) (layer F.Cu) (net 15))
 (segment (start 179.578 120.396) (end 185.166 120.396) (width 0.25) (layer F.Cu) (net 15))
 (segment (start 179.31892 120.65508) (end 179.578 120.396) (width 0.25) (layer F.Cu) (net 15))
 (segment (start 181.2798 125.7046) (end 181.2798 124.8918) (width 0.25) (layer F.Cu) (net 16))
 (segment (start 180.11902 123.73102) (end 180.11902 121.6406) (width 0.25) (layer F.Cu) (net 16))
 (segment (start 181.2798 124.8918) (end 180.11902 123.73102) (width 0.25) (layer F.Cu) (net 16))
 (segment (start 183.4388 125.7046) (end 183.4388 124.5108) (width 0.25) (layer F.Cu) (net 17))
 (segment (start 180.91912 123.26112) (end 180.91912 121.6406) (width 0.25) (layer F.Cu) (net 17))
 (segment (start 181.356 123.698) (end 180.91912 123.26112) (width 0.25) (layer F.Cu) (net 17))
 (segment (start 182.626 123.698) (end 181.356 123.698) (width 0.25) (layer F.Cu) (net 17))
 (segment (start 183.4388 124.5108) (end 182.626 123.698) (width 0.25) (layer F.Cu) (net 17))
 (segment (start 186.6773 125.7046) (end 186.6773 124.4473) (width 0.25) (layer F.Cu) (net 18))
 (segment (start 181.71922 122.79122) (end 181.71922 121.6406) (width 0.25) (layer F.Cu) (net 18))
 (segment (start 181.864 122.936) (end 181.71922 122.79122) (width 0.25) (layer F.Cu) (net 18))
 (segment (start 185.166 122.936) (end 181.864 122.936) (width 0.25) (layer F.Cu) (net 18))
 (segment (start 186.6773 124.4473) (end 185.166 122.936) (width 0.25) (layer F.Cu) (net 18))
 (segment (start 174.752 141.478) (end 174.752 140.97) (width 0.25) (layer F.Cu) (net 36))
 (segment (start 174.752 140.97) (end 176.53 139.192) (width 0.25) (layer F.Cu) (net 36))
 (segment (start 176.53 139.192) (end 176.53 134.26186) (width 0.25) (layer F.Cu) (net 36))
 (segment (start 191.516 104.14) (end 196.97446 104.14) (width 0.25) (layer F.Cu) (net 27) (status C00000))
 (segment (start 184.91708 112.98174) (end 186.73826 112.98174) (width 0.25) (layer F.Cu) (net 27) (status 400000))
 (segment (start 193.802 105.41) (end 192.532 104.14) (width 0.25) (layer F.Cu) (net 27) (status 800000))
 (segment (start 193.802 107.188) (end 193.802 105.41) (width 0.25) (layer F.Cu) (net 27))
 (segment (start 192.532 108.458) (end 193.802 107.188) (width 0.25) (layer F.Cu) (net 27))
 (segment (start 191.262 108.458) (end 192.532 108.458) (width 0.25) (layer F.Cu) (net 27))
 (segment (start 186.73826 112.98174) (end 191.262 108.458) (width 0.25) (layer F.Cu) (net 27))
 (segment (start 192.532 104.14) (end 191.516 104.14) (width 0.25) (layer F.Cu) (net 27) (status C00000)))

